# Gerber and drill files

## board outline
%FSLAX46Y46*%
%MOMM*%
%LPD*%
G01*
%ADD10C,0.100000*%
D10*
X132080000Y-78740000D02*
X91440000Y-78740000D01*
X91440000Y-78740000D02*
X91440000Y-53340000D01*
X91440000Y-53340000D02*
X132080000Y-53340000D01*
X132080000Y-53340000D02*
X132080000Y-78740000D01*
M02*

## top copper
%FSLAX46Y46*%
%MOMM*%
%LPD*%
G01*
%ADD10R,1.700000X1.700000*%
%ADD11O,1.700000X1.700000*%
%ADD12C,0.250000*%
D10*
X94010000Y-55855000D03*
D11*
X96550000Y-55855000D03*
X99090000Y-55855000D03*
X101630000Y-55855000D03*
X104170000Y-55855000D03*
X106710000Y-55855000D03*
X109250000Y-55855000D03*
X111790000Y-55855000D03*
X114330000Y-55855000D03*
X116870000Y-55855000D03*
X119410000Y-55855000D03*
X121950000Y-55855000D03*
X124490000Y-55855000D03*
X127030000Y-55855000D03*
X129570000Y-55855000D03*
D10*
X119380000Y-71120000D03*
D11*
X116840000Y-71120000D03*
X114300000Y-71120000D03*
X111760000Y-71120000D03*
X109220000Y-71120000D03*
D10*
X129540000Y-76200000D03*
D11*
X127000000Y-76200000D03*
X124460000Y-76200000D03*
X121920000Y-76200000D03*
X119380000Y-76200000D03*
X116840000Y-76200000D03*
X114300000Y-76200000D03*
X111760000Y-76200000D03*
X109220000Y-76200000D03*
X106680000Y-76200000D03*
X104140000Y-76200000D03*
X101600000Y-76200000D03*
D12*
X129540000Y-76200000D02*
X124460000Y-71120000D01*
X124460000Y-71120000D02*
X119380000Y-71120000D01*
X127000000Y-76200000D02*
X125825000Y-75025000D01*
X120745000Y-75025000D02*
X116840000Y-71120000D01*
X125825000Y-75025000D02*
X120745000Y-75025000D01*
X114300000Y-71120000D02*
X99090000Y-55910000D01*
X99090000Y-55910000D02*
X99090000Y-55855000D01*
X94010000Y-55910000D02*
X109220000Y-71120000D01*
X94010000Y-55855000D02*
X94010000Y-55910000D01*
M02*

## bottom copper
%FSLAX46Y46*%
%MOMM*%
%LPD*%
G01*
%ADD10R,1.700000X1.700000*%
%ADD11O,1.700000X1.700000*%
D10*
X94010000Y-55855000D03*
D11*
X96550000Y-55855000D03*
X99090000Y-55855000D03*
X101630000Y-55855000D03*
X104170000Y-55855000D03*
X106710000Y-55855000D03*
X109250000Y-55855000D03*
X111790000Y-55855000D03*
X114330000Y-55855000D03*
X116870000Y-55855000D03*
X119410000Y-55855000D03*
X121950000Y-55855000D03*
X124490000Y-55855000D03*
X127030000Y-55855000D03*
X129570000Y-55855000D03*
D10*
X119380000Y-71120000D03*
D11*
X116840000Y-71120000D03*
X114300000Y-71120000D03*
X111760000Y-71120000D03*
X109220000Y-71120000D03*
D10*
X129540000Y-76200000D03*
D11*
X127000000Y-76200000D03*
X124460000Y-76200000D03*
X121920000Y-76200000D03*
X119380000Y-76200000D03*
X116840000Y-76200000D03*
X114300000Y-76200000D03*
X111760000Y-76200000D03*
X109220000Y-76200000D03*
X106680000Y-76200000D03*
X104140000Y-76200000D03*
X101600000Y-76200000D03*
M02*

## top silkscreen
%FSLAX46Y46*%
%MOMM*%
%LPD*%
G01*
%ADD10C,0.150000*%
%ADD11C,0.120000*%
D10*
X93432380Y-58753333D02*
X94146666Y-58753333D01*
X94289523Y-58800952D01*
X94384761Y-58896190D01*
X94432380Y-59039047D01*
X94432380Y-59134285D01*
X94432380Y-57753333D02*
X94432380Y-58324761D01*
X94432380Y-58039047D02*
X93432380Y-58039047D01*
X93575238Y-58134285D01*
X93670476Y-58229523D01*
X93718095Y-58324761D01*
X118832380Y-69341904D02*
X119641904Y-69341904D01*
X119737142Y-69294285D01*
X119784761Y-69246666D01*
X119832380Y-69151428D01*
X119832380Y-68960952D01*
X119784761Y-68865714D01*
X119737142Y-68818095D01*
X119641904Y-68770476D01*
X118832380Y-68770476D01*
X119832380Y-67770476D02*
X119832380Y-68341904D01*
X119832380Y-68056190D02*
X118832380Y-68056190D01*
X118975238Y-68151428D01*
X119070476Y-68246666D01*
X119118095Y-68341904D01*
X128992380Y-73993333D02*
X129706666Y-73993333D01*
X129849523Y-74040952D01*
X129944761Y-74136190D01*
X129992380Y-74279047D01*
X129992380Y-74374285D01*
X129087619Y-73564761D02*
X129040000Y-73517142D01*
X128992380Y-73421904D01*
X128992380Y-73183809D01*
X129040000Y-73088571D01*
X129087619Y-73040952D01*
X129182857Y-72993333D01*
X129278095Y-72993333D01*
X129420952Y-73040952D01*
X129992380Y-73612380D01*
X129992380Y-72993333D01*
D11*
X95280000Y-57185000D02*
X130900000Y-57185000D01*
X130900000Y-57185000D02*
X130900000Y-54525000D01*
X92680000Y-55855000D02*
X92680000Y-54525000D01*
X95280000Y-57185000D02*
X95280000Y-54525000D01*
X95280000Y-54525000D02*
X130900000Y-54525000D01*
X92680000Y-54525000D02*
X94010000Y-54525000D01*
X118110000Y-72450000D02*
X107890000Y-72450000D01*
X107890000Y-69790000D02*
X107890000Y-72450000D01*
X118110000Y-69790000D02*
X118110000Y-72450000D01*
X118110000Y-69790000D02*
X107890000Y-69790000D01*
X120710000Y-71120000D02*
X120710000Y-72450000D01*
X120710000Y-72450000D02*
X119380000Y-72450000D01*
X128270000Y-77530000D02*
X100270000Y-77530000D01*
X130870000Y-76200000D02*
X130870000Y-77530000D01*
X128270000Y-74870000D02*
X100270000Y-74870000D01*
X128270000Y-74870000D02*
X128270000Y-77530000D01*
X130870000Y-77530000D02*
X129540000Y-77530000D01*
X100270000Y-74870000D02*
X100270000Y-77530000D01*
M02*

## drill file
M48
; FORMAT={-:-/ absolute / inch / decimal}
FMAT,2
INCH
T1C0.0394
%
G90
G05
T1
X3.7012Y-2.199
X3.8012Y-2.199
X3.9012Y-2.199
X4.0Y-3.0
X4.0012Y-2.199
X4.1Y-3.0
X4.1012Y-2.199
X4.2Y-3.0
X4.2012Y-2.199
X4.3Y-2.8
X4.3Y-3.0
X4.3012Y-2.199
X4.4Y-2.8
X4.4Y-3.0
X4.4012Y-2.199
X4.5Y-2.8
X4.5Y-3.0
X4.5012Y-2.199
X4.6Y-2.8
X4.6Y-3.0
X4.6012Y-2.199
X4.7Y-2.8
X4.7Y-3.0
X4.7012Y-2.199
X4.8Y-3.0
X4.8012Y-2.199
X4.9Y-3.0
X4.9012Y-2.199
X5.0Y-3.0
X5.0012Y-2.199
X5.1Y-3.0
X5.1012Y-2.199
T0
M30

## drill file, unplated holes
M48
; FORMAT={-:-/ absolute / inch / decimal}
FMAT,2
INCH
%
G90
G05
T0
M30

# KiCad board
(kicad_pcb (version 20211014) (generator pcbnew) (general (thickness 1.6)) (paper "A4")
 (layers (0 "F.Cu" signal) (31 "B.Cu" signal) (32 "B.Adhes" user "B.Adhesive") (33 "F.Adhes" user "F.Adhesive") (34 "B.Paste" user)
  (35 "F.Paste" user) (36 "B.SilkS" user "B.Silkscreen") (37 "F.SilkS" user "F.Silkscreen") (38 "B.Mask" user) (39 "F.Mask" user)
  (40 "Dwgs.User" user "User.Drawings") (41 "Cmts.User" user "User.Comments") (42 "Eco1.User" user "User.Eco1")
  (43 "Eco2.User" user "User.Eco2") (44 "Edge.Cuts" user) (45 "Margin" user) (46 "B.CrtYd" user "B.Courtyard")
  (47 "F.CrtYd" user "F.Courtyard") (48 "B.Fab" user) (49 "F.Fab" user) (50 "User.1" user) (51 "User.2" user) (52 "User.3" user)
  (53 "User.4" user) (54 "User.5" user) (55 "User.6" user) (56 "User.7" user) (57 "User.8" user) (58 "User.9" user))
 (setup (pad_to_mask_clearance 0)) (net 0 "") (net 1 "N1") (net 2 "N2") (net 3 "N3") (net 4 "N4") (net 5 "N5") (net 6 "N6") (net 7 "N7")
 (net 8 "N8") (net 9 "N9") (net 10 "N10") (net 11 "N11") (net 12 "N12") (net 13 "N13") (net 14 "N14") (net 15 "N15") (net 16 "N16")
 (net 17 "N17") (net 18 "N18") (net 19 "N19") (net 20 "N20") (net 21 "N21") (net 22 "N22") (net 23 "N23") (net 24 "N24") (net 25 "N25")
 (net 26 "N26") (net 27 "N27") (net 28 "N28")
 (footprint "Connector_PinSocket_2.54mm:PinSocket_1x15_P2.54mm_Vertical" (layer "F.Cu") (at 94.01 55.855 90)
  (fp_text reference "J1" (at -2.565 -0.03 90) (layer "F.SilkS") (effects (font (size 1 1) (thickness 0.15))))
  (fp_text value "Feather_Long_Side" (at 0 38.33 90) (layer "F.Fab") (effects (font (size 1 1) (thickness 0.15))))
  (fp_line (start -1.33 1.27) (end -1.33 36.89) (layer "F.SilkS") (width 0.12))
  (fp_line (start -1.33 36.89) (end 1.33 36.89) (layer "F.SilkS") (width 0.12))
  (fp_line (start 0 -1.33) (end 1.33 -1.33) (layer "F.SilkS") (width 0.12))
  (fp_line (start -1.33 1.27) (end 1.33 1.27) (layer "F.SilkS") (width 0.12))
  (fp_line (start 1.33 1.27) (end 1.33 36.89) (layer "F.SilkS") (width 0.12))
  (fp_line (start 1.33 -1.33) (end 1.33 0) (layer "F.SilkS") (width 0.12))
  (pad "1" thru_hole rect (at 0 0 90) (size 1.7 1.7) (drill 1) (layers *.Cu *.Mask) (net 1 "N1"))
  (pad "2" thru_hole oval (at 0 2.54 90) (size 1.7 1.7) (drill 1) (layers *.Cu *.Mask) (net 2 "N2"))
  (pad "3" thru_hole oval (at 0 5.08 90) (size 1.7 1.7) (drill 1) (layers *.Cu *.Mask) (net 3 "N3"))
  (pad "4" thru_hole oval (at 0 7.62 90) (size 1.7 1.7) (drill 1) (layers *.Cu *.Mask) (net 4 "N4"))
  (pad "5" thru_hole oval (at 0 10.16 90) (size 1.7 1.7) (drill 1) (layers *.Cu *.Mask) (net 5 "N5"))
  (pad "6" thru_hole oval (at 0 12.7 90) (size 1.7 1.7) (drill 1) (layers *.Cu *.Mask) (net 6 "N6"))
  (pad "7" thru_hole oval (at 0 15.24 90) (size 1.7 1.7) (drill 1) (layers *.Cu *.Mask) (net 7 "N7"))
  (pad "8" thru_hole oval (at 0 17.78 90) (size 1.7 1.7) (drill 1) (layers *.Cu *.Mask) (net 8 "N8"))
  (pad "9" thru_hole oval (at 0 20.32 90) (size 1.7 1.7) (drill 1) (layers *.Cu *.Mask) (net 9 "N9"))
  (pad "10" thru_hole oval (at 0 22.86 90) (size 1.7 1.7) (drill 1) (layers *.Cu *.Mask) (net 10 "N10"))
  (pad "11" thru_hole oval (at 0 25.4 90) (size 1.7 1.7) (drill 1) (layers *.Cu *.Mask) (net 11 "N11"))
  (pad "12" thru_hole oval (at 0 27.94 90) (size 1.7 1.7) (drill 1) (layers *.Cu *.Mask) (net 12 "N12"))
  (pad "13" thru_hole oval (at 0 30.48 90) (size 1.7 1.7) (drill 1) (layers *.Cu *.Mask) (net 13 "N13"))
  (pad "14" thru_hole oval (at 0 33.02 90) (size 1.7 1.7) (drill 1) (layers *.Cu *.Mask) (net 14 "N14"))
  (pad "15" thru_hole oval (at 0 35.56 90) (size 1.7 1.7) (drill 1) (layers *.Cu *.Mask) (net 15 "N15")))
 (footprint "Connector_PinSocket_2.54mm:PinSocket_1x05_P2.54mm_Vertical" (layer "F.Cu") (at 119.38 71.12 -90)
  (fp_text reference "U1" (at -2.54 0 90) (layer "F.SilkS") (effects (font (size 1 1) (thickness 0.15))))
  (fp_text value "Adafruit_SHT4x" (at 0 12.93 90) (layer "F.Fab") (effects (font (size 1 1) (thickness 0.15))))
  (fp_line (start 1.33 1.27) (end 1.33 11.49) (layer "F.SilkS") (width 0.12))
  (fp_line (start -1.33 11.49) (end 1.33 11.49) (layer "F.SilkS") (width 0.12))
  (fp_line (start -1.33 1.27) (end 1.33 1.27) (layer "F.SilkS") (width 0.12))
  (fp_line (start -1.33 1.27) (end -1.33 11.49) (layer "F.SilkS") (width 0.12))
  (fp_line (start 0 -1.33) (end 1.33 -1.33) (layer "F.SilkS") (width 0.12))
  (fp_line (start 1.33 -1.33) (end 1.33 0) (layer "F.SilkS") (width 0.12))
  (pad "1" thru_hole rect (at 0 0 270) (size 1.7 1.7) (drill 1) (layers *.Cu *.Mask) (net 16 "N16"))
  (pad "2" thru_hole oval (at 0 2.54 270) (size 1.7 1.7) (drill 1) (layers *.Cu *.Mask) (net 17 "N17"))
  (pad "3" thru_hole oval (at 0 5.08 270) (size 1.7 1.7) (drill 1) (layers *.Cu *.Mask) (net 3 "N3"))
  (pad "4" thru_hole oval (at 0 7.62 270) (size 1.7 1.7) (drill 1) (layers *.Cu *.Mask) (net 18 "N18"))
  (pad "5" thru_hole oval (at 0 10.16 270) (size 1.7 1.7) (drill 1) (layers *.Cu *.Mask) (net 1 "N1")))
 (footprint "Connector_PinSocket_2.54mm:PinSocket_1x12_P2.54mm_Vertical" (layer "F.Cu") (at 129.54 76.2 -90)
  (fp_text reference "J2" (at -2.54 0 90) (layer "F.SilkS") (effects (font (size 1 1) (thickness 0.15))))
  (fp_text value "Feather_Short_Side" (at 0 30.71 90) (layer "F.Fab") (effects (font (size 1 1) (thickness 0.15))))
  (fp_line (start 1.33 1.27) (end 1.33 29.27) (layer "F.SilkS") (width 0.12))
  (fp_line (start 0 -1.33) (end 1.33 -1.33) (layer "F.SilkS") (width 0.12))
  (fp_line (start -1.33 1.27) (end -1.33 29.27) (layer "F.SilkS") (width 0.12))
  (fp_line (start -1.33 1.27) (end 1.33 1.27) (layer "F.SilkS") (width 0.12))
  (fp_line (start 1.33 -1.33) (end 1.33 0) (layer "F.SilkS") (width 0.12))
  (fp_line (start -1.33 29.27) (end 1.33 29.27) (layer "F.SilkS") (width 0.12))
  (pad "1" thru_hole rect (at 0 0 270) (size 1.7 1.7) (drill 1) (layers *.Cu *.Mask) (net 16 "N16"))
  (pad "2" thru_hole oval (at 0 2.54 270) (size 1.7 1.7) (drill 1) (layers *.Cu *.Mask) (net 17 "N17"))
  (pad "3" thru_hole oval (at 0 5.08 270) (size 1.7 1.7) (drill 1) (layers *.Cu *.Mask) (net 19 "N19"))
  (pad "4" thru_hole oval (at 0 7.62 270) (size 1.7 1.7) (drill 1) (layers *.Cu *.Mask) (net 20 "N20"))
  (pad "5" thru_hole oval (at 0 10.16 270) (size 1.7 1.7) (drill 1) (layers *.Cu *.Mask) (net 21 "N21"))
  (pad "6" thru_hole oval (at 0 12.7 270) (size 1.7 1.7) (drill 1) (layers *.Cu *.Mask) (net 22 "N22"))
  (pad "7" thru_hole oval (at 0 15.24 270) (size 1.7 1.7) (drill 1) (layers *.Cu *.Mask) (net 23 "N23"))
  (pad "8" thru_hole oval (at 0 17.78 270) (size 1.7 1.7) (drill 1) (layers *.Cu *.Mask) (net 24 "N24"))
  (pad "9" thru_hole oval (at 0 20.32 270) (size 1.7 1.7) (drill 1) (layers *.Cu *.Mask) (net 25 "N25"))
  (pad "10" thru_hole oval (at 0 22.86 270) (size 1.7 1.7) (drill 1) (layers *.Cu *.Mask) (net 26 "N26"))
  (pad "11" thru_hole oval (at 0 25.4 270) (size 1.7 1.7) (drill 1) (layers *.Cu *.Mask) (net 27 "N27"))
  (pad "12" thru_hole oval (at 0 27.94 270) (size 1.7 1.7) (drill 1) (layers *.Cu *.Mask) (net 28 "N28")))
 (gr_rect (start 132.08 78.74) (end 91.44 53.34) (layer "Edge.Cuts") (width 0.1) (fill none))
 (segment (start 129.54 76.2) (end 124.46 71.12) (width 0.25) (layer "F.Cu") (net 16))
 (segment (start 124.46 71.12) (end 119.38 71.12) (width 0.25) (layer "F.Cu") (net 16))
 (segment (start 127 76.2) (end 125.825 75.025) (width 0.25) (layer "F.Cu") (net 17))
 (segment (start 120.745 75.025) (end 116.84 71.12) (width 0.25) (layer "F.Cu") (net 17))
 (segment (start 125.825 75.025) (end 120.745 75.025) (width 0.25) (layer "F.Cu") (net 17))
 (segment (start 114.3 71.12) (end 99.09 55.91) (width 0.25) (layer "F.Cu") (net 3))
 (segment (start 99.09 55.91) (end 99.09 55.855) (width 0.25) (layer "F.Cu") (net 3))
 (segment (start 94.01 55.91) (end 109.22 71.12) (width 0.25) (layer "F.Cu") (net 1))
 (segment (start 94.01 55.855) (end 94.01 55.91) (width 0.25) (layer "F.Cu") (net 1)))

